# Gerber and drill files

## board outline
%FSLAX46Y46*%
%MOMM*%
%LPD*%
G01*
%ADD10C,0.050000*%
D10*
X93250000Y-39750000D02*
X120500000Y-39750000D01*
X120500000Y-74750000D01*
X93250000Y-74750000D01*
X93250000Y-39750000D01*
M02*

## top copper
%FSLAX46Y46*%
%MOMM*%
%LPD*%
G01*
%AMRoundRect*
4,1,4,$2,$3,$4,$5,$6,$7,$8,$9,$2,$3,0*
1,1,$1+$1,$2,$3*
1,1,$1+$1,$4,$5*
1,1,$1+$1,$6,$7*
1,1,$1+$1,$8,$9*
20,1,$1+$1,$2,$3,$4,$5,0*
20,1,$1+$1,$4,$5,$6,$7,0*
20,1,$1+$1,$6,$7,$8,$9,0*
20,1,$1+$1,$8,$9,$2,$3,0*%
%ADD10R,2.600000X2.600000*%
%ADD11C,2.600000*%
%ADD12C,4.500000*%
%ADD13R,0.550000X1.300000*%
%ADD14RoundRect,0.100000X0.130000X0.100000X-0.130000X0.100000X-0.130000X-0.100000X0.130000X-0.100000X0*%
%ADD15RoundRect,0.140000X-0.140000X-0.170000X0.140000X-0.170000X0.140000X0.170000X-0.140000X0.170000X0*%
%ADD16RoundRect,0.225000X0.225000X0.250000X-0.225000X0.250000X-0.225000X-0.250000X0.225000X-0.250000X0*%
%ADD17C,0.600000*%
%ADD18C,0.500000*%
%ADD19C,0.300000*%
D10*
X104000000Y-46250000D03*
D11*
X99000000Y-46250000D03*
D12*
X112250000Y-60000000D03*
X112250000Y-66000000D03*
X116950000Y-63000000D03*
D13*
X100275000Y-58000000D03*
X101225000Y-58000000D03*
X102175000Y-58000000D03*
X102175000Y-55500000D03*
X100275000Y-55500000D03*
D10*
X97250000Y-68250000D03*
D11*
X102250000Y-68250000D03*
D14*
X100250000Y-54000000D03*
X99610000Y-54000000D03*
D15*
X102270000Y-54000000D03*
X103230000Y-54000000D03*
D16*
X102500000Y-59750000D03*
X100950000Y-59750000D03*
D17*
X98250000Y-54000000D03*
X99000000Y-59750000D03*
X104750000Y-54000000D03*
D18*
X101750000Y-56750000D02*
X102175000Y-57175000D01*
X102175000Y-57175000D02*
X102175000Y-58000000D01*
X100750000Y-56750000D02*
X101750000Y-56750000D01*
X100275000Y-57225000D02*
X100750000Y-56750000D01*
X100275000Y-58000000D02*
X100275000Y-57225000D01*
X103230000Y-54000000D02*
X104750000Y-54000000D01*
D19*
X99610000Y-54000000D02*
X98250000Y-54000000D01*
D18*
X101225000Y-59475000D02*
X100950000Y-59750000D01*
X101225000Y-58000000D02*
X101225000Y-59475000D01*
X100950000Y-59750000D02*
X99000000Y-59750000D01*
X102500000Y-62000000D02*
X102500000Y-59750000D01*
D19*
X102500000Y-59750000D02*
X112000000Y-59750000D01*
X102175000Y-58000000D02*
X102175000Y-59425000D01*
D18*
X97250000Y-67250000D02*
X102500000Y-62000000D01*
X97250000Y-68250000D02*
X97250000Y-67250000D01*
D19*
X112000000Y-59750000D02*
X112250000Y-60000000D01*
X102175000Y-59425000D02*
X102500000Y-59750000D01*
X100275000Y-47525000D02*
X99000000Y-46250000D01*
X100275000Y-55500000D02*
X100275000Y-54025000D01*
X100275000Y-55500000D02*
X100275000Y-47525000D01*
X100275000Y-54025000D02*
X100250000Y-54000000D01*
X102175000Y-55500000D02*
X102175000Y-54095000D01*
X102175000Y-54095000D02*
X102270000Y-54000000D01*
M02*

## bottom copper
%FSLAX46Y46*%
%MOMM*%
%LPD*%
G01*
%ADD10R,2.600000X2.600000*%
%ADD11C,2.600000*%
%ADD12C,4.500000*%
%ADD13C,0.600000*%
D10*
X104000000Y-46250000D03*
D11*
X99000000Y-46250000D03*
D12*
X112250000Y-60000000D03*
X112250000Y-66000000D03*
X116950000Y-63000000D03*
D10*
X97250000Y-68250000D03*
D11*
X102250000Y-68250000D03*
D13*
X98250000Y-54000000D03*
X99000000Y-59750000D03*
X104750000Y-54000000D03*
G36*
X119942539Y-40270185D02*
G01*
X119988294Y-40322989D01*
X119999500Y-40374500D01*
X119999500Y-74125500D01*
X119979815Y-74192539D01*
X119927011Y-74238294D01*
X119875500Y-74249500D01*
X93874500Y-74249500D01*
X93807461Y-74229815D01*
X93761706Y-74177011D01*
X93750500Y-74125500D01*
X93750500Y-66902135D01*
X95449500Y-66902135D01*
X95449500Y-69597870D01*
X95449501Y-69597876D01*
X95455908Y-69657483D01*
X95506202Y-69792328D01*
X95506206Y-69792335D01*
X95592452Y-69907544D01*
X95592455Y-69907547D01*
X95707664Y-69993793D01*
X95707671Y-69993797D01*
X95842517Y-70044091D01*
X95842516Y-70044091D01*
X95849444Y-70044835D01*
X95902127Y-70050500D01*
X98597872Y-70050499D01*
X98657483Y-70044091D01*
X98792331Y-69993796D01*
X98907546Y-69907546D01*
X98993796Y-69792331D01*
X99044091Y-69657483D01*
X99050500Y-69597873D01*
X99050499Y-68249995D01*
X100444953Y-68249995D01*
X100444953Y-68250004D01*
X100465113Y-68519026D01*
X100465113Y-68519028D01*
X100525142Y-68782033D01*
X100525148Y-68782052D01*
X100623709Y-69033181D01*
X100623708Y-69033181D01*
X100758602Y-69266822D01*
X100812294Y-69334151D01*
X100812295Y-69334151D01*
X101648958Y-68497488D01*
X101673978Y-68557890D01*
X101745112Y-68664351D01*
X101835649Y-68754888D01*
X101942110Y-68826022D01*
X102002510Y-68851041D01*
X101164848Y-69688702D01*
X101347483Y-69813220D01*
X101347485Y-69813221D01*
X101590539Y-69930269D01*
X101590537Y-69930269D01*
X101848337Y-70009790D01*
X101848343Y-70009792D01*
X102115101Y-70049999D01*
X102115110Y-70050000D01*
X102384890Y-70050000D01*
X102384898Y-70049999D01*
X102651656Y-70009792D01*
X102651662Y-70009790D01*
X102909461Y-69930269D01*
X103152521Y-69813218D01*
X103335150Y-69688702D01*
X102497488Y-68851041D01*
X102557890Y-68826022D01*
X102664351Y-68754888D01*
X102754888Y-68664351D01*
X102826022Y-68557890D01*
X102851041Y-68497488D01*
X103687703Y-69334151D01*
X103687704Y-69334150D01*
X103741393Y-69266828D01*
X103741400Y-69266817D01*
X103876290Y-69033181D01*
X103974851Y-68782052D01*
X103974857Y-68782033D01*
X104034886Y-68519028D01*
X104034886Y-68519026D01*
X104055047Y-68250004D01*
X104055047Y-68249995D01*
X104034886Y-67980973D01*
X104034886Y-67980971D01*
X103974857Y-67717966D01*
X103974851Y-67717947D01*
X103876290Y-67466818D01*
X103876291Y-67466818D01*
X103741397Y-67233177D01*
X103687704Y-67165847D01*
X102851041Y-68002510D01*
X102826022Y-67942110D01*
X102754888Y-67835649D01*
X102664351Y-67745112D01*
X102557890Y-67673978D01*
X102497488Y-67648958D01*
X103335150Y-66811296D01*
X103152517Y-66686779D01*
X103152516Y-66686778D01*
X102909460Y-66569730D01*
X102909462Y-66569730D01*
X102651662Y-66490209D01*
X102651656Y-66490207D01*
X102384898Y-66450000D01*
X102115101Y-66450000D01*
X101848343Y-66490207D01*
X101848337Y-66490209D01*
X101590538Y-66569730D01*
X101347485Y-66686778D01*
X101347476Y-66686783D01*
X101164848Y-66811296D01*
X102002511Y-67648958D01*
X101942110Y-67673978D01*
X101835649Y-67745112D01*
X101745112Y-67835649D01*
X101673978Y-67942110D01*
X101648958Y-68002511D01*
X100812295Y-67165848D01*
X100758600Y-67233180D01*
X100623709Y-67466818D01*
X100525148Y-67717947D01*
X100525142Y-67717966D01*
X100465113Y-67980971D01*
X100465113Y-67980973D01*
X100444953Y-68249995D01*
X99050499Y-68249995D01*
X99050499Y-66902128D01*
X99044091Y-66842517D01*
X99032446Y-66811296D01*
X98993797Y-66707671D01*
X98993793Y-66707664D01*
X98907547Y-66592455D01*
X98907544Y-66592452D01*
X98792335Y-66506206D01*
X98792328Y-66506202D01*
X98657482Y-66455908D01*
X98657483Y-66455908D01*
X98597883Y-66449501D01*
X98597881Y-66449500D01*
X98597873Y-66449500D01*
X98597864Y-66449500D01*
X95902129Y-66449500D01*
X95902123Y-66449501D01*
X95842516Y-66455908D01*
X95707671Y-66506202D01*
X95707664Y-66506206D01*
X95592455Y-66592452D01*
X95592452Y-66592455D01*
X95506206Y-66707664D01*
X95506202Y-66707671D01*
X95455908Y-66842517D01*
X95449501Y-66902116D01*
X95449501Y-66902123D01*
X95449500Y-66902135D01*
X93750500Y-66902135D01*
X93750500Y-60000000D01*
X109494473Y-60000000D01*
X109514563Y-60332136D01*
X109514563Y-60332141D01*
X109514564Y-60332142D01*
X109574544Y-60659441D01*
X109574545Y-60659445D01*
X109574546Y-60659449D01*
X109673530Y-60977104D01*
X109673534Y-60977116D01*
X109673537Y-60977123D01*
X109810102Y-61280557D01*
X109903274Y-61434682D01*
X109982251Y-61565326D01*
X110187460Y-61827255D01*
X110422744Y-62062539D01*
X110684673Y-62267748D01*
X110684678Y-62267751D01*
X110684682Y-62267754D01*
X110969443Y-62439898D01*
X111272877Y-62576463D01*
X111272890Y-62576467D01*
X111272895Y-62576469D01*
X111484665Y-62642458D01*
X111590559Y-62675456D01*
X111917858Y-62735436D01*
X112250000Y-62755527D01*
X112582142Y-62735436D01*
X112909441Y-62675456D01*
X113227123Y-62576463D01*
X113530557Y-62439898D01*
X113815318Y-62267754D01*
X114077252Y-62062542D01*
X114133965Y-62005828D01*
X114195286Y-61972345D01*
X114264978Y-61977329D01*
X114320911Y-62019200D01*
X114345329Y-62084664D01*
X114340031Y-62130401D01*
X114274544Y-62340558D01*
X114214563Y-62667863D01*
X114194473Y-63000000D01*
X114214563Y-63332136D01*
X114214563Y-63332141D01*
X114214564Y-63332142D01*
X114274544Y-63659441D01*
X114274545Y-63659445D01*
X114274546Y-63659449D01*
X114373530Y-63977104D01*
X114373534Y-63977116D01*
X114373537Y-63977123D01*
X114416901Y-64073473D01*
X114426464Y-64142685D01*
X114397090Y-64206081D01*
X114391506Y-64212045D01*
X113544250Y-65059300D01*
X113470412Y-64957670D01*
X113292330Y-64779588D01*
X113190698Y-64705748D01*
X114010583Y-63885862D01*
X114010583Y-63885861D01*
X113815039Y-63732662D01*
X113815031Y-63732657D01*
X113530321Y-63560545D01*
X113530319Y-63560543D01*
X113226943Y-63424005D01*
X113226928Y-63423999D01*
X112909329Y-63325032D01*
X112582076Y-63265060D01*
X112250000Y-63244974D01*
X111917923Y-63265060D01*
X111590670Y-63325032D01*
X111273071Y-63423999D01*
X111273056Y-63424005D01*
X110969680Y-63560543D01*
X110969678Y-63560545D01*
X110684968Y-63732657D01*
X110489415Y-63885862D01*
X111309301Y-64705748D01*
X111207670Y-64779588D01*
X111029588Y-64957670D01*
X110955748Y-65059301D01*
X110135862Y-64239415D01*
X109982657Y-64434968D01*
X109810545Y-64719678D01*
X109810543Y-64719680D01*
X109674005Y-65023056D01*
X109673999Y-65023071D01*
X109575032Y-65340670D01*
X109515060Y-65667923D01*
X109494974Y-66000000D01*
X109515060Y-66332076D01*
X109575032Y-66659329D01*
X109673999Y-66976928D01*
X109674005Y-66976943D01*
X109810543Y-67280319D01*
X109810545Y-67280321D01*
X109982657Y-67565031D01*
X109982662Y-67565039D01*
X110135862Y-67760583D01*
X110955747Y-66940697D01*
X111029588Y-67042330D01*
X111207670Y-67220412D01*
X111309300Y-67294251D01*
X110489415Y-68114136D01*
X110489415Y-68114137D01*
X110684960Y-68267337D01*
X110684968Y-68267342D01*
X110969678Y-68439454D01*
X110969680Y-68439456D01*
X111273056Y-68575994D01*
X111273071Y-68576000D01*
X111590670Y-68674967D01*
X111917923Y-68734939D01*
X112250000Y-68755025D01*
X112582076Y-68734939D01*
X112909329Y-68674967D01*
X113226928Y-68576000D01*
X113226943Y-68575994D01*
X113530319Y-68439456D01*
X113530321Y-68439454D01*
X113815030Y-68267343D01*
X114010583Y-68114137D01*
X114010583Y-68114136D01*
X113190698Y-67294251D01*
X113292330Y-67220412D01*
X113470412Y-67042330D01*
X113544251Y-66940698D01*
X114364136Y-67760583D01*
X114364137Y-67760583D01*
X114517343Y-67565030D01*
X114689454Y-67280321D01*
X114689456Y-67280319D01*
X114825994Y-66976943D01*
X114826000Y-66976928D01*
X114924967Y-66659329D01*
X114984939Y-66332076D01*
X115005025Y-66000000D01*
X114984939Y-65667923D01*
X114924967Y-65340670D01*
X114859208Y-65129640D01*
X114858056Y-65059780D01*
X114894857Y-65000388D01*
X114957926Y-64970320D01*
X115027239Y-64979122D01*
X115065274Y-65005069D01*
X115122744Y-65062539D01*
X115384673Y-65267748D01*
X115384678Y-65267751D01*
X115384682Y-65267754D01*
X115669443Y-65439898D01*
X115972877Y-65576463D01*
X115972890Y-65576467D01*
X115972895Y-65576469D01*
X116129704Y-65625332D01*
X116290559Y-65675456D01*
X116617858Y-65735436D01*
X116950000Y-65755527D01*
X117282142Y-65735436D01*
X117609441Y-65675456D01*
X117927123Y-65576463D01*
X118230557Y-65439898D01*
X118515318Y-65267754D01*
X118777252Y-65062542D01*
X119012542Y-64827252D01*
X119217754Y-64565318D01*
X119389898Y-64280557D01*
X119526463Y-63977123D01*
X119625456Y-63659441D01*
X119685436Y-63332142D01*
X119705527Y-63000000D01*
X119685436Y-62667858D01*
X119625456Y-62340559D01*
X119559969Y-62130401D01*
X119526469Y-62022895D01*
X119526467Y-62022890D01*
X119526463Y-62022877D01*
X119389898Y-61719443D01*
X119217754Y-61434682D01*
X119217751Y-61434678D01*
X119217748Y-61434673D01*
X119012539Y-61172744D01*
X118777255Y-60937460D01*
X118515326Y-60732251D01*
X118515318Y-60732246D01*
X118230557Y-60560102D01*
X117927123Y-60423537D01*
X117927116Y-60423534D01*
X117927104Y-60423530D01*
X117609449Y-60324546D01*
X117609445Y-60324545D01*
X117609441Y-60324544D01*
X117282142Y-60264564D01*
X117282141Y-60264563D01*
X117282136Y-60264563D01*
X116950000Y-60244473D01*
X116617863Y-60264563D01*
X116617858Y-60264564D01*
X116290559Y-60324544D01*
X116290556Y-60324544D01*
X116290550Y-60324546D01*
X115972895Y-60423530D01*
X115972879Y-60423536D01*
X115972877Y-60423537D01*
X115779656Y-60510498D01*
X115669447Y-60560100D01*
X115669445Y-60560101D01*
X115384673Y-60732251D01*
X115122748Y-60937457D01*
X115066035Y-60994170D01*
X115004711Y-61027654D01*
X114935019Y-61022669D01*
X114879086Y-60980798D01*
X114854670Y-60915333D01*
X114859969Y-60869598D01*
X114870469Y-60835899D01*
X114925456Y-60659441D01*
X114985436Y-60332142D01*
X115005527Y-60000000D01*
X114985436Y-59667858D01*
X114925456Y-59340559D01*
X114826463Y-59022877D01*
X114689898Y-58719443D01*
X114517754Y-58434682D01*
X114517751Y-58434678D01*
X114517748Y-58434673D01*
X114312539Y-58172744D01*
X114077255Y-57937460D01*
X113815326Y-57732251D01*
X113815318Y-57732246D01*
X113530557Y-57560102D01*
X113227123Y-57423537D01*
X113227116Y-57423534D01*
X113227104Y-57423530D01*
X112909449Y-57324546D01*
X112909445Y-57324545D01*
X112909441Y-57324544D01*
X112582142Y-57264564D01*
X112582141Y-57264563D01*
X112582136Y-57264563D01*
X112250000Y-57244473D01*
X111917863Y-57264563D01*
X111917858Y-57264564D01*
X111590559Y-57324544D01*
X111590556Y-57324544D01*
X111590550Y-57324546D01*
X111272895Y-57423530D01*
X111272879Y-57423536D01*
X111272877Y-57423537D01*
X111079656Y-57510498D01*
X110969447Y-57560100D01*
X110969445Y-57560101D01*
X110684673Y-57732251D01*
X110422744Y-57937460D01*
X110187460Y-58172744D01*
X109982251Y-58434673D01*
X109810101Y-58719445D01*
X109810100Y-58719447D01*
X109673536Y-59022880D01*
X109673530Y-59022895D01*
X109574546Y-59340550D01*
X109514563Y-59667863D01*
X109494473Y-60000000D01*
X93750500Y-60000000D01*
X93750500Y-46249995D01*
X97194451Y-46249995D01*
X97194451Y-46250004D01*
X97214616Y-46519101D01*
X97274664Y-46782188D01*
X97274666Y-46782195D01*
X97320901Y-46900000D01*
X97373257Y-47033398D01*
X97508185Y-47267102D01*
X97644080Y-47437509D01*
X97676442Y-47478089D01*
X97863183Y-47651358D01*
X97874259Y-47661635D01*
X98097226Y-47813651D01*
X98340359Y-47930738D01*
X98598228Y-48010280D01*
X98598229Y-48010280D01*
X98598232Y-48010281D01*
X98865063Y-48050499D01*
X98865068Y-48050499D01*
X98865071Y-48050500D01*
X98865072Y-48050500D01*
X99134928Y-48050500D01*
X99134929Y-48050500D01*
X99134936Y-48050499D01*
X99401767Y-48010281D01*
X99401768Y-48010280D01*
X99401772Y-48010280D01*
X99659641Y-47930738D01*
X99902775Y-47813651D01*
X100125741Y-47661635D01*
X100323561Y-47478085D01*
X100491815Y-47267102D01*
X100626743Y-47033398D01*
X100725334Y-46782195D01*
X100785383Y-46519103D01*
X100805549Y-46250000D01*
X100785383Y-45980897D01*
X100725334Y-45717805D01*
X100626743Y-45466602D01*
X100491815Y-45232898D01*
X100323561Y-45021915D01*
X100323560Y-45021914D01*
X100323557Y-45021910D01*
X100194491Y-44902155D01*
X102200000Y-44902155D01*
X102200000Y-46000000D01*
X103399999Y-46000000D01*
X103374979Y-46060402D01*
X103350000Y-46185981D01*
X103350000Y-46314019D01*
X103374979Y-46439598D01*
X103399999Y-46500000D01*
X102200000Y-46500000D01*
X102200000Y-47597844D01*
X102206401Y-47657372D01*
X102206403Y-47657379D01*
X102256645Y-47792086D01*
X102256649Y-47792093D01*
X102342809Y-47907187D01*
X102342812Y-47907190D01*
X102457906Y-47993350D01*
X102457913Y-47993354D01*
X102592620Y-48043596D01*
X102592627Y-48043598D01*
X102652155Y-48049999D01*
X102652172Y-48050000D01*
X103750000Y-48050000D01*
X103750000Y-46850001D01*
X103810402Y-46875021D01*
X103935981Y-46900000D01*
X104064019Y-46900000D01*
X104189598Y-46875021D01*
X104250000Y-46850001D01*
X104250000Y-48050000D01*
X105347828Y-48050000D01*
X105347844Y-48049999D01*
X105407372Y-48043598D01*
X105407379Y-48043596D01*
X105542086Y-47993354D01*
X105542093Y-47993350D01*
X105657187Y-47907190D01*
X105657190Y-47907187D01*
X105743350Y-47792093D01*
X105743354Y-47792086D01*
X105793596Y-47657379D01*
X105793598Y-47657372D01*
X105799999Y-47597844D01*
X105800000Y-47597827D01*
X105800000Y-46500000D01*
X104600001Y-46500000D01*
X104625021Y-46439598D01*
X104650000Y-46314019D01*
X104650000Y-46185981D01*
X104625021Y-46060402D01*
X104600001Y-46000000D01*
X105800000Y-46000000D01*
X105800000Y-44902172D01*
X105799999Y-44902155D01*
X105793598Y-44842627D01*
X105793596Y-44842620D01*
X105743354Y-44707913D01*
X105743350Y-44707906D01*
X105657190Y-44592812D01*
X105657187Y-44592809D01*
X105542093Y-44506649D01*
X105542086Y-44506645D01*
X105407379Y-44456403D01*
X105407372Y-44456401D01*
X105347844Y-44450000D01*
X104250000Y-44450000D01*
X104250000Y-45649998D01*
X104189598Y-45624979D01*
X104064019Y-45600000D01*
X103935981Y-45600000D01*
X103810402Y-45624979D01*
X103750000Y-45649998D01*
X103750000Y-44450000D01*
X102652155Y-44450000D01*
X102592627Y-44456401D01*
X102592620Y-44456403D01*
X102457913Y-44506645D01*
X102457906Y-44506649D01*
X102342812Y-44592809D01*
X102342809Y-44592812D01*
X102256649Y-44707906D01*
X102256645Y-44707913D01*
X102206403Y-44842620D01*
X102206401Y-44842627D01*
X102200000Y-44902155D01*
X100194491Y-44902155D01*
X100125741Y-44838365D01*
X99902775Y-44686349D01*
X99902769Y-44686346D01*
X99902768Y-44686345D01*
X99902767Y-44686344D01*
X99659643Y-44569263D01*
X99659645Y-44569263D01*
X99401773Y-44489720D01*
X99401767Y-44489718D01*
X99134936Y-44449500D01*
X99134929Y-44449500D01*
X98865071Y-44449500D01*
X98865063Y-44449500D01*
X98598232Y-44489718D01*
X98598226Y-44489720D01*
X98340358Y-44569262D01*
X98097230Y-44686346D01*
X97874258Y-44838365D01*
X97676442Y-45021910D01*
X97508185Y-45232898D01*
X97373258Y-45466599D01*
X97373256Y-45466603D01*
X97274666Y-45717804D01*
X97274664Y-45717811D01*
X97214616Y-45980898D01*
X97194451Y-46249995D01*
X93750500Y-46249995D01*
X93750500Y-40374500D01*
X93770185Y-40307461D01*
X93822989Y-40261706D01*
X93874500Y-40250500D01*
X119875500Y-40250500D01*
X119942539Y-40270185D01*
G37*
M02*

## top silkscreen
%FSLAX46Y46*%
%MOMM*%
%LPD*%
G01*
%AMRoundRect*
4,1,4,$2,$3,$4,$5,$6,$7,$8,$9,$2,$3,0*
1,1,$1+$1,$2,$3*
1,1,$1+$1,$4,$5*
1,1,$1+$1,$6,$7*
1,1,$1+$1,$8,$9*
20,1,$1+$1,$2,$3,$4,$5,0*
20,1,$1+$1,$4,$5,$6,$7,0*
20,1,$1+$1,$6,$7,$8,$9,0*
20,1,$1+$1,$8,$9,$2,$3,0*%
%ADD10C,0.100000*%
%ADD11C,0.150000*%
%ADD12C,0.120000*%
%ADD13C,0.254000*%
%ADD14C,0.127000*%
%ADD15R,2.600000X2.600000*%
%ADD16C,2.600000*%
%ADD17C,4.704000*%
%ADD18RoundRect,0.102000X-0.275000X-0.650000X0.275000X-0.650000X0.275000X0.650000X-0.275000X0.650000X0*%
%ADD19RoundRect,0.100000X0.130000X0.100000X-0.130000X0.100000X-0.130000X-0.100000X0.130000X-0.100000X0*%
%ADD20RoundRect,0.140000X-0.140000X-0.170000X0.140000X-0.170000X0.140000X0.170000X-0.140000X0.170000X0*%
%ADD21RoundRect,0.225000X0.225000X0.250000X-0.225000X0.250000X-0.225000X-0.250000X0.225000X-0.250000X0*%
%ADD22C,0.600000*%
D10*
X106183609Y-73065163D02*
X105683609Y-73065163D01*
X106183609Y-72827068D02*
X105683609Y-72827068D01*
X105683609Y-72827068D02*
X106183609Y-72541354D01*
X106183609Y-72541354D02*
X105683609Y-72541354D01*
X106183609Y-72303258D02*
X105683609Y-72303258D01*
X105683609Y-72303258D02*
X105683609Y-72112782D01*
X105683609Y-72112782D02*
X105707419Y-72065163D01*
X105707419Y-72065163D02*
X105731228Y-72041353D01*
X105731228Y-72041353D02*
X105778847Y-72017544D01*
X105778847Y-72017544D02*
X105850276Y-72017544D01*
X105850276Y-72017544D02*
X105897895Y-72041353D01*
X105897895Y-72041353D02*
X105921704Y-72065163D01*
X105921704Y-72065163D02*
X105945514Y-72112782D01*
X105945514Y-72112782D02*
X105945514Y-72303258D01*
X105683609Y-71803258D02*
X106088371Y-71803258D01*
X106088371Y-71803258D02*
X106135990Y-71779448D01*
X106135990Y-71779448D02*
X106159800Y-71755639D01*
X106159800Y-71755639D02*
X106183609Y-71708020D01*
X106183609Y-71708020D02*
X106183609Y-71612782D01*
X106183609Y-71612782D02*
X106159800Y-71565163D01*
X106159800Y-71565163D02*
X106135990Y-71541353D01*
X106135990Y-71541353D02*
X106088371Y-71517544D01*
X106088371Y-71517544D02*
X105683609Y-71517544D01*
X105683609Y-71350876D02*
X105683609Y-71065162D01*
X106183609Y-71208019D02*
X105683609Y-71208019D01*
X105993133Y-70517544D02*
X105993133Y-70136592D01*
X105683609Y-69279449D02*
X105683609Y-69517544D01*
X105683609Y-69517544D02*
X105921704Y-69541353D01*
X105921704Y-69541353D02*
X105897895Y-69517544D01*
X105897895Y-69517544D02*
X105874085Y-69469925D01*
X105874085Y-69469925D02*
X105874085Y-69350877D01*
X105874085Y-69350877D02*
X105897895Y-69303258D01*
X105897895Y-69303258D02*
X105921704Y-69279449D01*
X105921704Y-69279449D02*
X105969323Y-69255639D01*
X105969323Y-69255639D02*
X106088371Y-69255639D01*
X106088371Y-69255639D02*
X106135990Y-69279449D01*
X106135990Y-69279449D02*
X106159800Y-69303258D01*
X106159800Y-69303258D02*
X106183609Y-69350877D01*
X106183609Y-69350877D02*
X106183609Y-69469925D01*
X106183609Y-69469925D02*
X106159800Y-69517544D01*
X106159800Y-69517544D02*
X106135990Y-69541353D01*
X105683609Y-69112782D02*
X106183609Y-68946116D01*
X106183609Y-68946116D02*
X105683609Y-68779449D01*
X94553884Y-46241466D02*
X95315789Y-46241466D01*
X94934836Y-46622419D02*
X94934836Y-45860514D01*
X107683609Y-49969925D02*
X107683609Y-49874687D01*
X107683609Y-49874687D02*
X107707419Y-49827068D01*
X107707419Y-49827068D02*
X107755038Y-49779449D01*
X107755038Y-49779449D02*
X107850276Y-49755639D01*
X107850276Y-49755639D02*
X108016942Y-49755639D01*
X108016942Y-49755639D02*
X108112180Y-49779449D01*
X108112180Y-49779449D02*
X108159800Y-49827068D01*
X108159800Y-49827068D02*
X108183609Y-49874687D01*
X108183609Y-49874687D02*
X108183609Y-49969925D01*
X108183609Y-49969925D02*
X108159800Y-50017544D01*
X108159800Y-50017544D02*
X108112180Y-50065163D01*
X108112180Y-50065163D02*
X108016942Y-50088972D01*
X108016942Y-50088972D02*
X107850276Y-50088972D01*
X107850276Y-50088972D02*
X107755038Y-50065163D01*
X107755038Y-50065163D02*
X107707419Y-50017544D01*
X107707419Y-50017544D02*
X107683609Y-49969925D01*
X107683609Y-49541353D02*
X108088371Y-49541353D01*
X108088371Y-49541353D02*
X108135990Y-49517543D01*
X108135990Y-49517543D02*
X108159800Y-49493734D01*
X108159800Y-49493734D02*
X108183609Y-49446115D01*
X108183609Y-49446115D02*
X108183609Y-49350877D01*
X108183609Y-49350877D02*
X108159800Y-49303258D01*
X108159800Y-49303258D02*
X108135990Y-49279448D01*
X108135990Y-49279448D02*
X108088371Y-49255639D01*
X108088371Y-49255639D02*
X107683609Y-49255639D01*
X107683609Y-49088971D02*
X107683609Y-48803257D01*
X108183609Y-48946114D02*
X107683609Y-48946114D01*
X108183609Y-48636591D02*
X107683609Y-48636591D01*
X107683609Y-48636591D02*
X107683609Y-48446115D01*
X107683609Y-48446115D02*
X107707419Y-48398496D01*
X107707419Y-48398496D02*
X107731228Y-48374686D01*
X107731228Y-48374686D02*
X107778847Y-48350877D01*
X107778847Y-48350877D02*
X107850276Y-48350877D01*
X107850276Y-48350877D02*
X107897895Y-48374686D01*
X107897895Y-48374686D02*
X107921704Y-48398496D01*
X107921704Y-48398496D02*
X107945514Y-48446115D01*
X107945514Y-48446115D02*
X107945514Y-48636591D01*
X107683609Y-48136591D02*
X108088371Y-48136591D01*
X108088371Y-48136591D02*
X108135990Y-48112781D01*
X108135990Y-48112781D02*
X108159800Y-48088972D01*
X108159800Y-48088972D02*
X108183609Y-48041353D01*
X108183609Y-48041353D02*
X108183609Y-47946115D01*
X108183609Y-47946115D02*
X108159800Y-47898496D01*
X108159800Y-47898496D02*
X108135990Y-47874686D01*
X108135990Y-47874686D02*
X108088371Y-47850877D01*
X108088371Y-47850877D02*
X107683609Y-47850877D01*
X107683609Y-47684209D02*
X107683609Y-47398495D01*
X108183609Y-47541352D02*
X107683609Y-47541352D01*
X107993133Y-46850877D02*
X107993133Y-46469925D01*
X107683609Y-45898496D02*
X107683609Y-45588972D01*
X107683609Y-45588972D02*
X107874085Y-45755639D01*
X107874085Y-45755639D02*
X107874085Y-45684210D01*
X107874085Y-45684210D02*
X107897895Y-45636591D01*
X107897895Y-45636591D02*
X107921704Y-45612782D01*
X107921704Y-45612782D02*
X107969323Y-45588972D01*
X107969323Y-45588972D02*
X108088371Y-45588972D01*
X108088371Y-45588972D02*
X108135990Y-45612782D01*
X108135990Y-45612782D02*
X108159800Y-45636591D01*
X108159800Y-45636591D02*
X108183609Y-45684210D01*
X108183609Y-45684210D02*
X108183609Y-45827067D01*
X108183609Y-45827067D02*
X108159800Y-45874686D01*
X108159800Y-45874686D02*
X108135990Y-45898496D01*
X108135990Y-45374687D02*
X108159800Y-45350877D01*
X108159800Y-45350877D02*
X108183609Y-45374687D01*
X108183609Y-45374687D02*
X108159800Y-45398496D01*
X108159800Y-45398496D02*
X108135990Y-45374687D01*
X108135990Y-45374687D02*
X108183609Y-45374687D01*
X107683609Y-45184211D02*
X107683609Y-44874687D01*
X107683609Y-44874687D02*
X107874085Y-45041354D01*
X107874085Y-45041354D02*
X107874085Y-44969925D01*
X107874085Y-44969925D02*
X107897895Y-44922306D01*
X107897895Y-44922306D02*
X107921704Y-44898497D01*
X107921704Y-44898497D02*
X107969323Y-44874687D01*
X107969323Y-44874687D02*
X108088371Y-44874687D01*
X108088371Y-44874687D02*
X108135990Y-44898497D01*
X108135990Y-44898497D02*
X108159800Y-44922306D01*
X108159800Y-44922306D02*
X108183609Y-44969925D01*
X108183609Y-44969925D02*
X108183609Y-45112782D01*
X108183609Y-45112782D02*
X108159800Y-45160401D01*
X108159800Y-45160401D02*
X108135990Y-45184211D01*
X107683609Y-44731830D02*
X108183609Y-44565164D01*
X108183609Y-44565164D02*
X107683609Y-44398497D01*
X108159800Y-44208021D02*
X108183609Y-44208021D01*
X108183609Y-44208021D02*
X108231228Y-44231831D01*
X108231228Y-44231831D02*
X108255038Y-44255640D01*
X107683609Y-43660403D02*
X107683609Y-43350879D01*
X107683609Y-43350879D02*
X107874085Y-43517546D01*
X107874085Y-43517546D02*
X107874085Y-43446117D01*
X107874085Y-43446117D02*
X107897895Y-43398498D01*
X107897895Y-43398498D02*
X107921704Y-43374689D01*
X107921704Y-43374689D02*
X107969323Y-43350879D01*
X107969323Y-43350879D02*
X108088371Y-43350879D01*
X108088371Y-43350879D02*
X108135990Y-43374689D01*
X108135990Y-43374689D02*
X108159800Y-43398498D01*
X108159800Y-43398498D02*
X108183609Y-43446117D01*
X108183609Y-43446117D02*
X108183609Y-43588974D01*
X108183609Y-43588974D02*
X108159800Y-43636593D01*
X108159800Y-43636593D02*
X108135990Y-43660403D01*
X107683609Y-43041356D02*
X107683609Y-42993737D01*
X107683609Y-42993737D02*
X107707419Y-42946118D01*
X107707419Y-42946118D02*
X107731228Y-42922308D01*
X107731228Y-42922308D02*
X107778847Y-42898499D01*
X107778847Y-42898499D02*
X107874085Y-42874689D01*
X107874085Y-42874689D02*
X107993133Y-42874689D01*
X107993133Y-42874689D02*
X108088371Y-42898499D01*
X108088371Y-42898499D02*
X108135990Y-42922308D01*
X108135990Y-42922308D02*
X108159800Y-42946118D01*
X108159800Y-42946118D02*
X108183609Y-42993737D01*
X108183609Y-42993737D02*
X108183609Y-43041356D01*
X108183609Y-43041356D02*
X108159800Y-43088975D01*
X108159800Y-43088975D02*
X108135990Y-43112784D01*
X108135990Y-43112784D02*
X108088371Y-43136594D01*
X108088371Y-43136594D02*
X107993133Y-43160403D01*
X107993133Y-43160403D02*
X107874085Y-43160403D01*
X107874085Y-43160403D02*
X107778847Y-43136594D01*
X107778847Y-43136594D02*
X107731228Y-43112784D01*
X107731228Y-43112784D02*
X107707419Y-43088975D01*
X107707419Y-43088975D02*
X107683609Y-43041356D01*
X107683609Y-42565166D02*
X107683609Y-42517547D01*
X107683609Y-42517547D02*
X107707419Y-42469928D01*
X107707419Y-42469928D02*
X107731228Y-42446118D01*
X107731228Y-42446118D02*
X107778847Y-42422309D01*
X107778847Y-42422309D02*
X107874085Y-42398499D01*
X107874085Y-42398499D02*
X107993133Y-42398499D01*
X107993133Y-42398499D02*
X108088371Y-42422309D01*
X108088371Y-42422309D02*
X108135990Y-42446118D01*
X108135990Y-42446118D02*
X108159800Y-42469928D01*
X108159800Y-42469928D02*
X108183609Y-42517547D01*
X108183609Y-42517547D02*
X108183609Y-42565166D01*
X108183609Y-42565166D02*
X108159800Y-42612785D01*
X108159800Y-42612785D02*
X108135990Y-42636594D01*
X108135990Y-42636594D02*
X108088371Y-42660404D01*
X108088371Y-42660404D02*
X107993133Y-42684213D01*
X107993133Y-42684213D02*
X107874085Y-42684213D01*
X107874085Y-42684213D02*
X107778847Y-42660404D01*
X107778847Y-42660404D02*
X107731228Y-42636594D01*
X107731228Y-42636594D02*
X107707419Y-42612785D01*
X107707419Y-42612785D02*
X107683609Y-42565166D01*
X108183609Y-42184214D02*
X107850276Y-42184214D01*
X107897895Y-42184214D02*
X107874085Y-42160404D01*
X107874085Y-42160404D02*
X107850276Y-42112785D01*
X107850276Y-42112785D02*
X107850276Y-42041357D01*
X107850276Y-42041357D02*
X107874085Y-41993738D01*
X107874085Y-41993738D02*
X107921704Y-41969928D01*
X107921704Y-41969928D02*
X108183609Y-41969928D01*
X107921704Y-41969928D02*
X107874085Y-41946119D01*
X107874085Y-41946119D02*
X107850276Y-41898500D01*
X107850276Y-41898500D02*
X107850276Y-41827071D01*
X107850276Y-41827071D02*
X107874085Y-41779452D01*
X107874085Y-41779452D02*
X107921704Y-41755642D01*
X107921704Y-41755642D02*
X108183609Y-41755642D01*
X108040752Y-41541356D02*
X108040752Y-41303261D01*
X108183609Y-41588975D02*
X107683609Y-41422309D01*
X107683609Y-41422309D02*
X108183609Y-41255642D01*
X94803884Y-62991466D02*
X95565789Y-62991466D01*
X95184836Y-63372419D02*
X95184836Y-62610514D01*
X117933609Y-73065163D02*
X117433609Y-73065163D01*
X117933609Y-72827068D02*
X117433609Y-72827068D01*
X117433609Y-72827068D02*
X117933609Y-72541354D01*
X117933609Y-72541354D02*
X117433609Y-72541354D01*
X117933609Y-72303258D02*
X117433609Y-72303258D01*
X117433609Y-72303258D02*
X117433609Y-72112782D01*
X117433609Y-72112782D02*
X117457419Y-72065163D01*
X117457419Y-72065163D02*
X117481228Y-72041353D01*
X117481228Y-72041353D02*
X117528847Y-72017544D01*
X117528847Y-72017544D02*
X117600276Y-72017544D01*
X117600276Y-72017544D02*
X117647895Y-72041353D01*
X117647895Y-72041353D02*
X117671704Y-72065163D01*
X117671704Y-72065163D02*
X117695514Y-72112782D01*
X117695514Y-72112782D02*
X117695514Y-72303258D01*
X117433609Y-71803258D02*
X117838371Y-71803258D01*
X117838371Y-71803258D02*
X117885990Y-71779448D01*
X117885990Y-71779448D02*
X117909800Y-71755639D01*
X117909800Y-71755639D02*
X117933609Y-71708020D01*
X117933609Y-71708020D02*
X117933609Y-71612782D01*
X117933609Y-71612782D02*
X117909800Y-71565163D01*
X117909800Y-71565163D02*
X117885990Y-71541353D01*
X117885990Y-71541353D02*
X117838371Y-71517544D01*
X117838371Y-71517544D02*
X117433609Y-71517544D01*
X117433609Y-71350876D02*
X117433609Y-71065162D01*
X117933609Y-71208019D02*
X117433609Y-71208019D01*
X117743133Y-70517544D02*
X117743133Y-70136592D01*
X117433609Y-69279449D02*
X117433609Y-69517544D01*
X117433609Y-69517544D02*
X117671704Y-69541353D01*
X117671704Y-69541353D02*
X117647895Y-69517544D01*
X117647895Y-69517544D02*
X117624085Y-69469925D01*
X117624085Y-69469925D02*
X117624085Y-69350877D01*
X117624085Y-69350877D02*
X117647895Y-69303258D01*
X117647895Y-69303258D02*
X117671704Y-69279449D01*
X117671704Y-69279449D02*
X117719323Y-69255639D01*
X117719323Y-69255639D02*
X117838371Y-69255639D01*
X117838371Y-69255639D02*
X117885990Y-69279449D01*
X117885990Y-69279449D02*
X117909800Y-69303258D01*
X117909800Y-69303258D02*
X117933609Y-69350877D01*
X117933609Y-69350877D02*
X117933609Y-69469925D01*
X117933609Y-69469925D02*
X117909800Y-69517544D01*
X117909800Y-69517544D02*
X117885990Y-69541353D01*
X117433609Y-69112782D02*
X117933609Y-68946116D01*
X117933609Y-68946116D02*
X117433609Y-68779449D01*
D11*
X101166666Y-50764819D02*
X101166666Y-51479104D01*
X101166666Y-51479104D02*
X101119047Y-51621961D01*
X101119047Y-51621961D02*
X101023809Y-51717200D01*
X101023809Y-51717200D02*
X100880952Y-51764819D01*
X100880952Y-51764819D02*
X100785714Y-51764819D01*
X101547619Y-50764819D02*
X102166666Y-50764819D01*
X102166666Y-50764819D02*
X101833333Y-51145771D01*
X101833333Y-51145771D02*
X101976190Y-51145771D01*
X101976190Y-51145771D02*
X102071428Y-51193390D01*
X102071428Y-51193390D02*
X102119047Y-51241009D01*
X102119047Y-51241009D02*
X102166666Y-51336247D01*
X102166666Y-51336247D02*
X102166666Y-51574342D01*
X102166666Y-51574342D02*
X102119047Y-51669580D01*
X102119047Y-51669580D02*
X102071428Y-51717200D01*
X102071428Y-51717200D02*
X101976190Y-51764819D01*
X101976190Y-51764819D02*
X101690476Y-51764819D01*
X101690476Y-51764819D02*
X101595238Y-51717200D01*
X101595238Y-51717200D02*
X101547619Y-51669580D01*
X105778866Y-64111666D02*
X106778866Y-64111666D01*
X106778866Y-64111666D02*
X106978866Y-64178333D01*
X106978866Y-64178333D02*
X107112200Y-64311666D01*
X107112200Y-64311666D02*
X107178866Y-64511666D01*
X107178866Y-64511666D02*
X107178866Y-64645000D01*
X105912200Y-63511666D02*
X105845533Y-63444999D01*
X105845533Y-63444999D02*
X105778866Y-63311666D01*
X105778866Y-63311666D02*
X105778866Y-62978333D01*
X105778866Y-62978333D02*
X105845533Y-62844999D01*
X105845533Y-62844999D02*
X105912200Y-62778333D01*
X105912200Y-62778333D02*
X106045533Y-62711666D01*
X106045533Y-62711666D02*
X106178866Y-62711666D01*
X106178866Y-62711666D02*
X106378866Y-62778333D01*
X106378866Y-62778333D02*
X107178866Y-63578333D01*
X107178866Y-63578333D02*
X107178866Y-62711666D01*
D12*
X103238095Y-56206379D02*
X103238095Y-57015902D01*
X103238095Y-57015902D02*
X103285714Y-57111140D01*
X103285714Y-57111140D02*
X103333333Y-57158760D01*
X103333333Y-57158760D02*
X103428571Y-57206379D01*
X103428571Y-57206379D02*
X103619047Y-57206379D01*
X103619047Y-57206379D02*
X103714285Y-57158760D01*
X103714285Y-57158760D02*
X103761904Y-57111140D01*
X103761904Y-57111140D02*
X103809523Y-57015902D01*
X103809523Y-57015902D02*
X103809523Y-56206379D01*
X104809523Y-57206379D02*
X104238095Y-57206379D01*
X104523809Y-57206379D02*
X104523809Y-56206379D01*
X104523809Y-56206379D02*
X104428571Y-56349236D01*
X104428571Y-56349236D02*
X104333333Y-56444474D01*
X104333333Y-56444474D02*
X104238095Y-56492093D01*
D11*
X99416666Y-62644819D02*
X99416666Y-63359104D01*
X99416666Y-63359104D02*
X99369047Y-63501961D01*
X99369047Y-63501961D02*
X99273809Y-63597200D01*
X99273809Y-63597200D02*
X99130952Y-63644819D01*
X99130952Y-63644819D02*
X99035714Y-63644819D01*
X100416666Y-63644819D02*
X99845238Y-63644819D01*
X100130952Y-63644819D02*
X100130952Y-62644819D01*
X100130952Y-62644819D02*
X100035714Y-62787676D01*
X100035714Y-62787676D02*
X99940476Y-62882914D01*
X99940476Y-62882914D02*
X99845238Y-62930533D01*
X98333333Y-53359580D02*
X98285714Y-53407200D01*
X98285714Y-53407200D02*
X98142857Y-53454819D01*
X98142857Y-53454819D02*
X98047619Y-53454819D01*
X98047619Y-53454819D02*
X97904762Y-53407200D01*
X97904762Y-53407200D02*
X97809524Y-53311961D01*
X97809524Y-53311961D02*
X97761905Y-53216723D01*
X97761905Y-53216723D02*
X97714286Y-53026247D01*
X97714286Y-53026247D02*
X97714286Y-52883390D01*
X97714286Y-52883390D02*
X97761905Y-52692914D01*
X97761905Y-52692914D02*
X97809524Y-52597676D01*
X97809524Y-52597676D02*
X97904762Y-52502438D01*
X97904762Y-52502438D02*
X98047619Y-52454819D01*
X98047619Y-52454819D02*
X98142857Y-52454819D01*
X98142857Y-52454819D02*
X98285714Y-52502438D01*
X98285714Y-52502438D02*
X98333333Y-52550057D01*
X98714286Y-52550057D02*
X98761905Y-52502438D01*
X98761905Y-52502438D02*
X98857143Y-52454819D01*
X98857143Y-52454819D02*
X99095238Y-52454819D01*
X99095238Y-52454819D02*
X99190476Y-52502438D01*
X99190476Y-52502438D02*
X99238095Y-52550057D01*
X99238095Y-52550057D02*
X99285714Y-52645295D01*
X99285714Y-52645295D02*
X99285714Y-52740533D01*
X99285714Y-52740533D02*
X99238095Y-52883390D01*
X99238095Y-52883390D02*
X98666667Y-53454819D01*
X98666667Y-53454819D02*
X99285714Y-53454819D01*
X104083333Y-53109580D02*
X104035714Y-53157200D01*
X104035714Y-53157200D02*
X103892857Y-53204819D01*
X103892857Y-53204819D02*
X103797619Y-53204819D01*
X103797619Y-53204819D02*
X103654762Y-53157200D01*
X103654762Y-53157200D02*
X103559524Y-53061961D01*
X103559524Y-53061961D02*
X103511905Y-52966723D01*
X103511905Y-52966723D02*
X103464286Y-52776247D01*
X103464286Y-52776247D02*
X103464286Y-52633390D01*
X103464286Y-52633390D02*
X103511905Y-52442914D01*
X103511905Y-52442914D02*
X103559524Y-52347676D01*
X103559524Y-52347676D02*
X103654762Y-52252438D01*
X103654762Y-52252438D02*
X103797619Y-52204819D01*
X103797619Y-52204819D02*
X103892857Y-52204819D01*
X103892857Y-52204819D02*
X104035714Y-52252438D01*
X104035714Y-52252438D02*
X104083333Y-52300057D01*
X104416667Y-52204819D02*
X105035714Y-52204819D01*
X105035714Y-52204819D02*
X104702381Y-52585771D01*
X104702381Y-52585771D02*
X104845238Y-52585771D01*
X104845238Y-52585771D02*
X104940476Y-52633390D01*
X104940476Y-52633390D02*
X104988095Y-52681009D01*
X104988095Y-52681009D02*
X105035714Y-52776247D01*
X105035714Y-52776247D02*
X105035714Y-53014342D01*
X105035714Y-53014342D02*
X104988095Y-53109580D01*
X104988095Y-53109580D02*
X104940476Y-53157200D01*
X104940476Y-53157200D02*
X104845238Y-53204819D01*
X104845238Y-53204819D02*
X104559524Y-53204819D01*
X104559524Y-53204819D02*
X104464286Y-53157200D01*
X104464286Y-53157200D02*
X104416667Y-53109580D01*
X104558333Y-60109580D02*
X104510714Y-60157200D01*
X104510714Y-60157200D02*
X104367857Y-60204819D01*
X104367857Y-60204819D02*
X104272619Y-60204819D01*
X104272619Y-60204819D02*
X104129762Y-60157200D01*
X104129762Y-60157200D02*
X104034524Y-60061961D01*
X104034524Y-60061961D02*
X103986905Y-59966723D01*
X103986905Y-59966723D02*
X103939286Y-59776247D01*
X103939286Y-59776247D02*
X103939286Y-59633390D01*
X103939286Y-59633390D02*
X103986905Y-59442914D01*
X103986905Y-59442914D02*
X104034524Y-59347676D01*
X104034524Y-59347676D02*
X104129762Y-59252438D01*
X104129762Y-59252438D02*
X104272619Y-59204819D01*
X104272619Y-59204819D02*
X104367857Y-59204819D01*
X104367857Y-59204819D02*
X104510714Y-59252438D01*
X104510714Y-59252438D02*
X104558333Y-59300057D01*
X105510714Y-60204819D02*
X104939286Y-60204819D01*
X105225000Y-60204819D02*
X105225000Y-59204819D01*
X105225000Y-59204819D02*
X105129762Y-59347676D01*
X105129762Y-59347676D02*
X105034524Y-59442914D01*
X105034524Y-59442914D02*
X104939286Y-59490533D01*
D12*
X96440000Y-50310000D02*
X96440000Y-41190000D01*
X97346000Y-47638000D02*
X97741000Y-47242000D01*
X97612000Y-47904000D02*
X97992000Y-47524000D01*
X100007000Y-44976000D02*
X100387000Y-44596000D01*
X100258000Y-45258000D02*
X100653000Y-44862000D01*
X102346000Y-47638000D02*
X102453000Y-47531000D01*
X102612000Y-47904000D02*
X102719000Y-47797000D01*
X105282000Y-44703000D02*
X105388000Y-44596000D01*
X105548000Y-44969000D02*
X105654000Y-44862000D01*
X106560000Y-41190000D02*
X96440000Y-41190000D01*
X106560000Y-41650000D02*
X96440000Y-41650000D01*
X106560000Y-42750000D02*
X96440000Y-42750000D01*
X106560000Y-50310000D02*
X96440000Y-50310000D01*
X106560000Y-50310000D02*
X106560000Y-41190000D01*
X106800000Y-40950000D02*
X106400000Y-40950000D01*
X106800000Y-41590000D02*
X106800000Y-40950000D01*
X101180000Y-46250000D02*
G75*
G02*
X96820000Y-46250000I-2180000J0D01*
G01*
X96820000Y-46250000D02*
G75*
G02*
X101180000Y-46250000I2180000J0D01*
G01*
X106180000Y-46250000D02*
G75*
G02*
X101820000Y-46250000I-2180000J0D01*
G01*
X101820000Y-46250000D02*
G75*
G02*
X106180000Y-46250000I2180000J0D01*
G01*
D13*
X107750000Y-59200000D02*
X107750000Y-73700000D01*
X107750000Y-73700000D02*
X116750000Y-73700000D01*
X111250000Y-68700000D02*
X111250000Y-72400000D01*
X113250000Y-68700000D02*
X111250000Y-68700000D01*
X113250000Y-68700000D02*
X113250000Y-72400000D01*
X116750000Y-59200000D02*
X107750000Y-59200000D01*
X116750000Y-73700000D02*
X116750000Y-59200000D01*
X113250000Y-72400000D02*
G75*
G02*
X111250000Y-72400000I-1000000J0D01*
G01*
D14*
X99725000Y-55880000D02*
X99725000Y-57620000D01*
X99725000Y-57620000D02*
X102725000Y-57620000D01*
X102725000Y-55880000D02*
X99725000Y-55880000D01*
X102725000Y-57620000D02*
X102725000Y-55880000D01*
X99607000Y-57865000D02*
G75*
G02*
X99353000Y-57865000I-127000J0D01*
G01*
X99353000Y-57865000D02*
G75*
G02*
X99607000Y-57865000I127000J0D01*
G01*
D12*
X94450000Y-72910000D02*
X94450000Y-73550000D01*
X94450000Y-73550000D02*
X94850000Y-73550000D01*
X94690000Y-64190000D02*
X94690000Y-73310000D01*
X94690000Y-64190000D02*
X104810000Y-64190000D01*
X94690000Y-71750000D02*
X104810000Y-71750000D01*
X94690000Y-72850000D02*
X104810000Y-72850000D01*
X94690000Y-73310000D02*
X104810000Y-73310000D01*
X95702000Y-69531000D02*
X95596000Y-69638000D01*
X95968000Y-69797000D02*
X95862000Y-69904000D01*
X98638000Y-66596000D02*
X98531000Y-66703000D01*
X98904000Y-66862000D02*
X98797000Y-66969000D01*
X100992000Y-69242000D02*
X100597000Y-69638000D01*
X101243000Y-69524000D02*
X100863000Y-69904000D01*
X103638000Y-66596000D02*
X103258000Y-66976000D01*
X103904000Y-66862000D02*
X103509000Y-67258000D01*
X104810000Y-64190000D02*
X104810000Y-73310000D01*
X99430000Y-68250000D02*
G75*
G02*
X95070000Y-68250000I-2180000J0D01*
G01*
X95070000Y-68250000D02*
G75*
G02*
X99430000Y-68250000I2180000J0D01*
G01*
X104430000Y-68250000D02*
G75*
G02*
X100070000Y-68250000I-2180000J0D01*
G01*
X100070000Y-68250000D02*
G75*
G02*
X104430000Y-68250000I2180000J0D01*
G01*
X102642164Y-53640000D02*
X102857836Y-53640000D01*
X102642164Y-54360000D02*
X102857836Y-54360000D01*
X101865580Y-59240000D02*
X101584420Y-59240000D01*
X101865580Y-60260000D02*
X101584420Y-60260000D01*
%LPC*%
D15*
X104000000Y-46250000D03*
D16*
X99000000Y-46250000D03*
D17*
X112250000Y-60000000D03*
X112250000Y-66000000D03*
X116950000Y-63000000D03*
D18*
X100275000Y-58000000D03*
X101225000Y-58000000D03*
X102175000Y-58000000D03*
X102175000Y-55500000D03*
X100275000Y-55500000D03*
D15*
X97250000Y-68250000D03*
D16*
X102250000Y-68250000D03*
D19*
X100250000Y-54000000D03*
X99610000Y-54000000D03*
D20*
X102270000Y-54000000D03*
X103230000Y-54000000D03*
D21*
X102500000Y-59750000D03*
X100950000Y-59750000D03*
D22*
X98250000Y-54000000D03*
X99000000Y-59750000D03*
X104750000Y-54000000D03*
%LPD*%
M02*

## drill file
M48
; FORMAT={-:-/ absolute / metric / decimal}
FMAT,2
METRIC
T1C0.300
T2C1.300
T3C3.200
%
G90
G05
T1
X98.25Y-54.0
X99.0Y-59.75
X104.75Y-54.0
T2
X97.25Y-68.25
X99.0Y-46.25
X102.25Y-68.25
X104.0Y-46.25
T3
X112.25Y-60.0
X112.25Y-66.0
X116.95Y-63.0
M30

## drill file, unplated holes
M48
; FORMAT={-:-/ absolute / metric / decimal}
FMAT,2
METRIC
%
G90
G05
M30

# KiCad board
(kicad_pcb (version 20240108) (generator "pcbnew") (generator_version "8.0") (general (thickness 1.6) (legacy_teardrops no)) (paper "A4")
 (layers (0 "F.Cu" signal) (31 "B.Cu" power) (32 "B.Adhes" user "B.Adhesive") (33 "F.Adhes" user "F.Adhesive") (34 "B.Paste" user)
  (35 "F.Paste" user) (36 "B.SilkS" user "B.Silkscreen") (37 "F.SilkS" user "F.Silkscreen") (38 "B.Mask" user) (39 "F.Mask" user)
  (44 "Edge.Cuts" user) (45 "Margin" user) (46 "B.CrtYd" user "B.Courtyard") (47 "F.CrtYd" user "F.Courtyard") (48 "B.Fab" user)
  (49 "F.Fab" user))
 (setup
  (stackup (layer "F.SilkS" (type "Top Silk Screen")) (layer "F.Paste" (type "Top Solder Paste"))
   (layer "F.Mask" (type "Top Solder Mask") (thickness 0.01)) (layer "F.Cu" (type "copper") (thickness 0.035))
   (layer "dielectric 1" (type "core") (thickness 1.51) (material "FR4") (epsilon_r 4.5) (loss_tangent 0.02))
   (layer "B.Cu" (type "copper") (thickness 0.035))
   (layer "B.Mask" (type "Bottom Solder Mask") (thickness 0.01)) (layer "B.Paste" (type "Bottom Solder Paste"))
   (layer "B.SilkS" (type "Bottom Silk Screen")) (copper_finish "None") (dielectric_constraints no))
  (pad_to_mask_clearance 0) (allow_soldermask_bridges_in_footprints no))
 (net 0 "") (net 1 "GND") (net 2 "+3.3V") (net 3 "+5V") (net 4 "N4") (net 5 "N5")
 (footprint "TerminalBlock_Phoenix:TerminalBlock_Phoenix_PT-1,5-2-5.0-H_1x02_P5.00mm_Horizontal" (layer "F.Cu") (at 104 46.25 180)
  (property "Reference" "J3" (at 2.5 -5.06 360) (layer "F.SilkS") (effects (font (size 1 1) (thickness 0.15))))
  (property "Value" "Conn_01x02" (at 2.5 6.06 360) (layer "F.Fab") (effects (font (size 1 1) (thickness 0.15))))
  (fp_line (start 7.56 -4.06) (end 7.56 5.06) (stroke (width 0.12) (type solid)) (layer "F.SilkS"))
  (fp_line (start 6.654 -1.388) (end 6.259 -0.992) (stroke (width 0.12) (type solid)) (layer "F.SilkS"))
  (fp_line (start 6.388 -1.654) (end 6.008 -1.274) (stroke (width 0.12) (type solid)) (layer "F.SilkS"))
  (fp_line (start 3.993 1.274) (end 3.613 1.654) (stroke (width 0.12) (type solid)) (layer "F.SilkS"))
  (fp_line (start 3.742 0.992) (end 3.347 1.388) (stroke (width 0.12) (type solid)) (layer "F.SilkS"))
  (fp_line (start 1.654 -1.388) (end 1.547 -1.281) (stroke (width 0.12) (type solid)) (layer "F.SilkS"))
  (fp_line (start 1.388 -1.654) (end 1.281 -1.547) (stroke (width 0.12) (type solid)) (layer "F.SilkS"))
  (fp_line (start -1.282 1.547) (end -1.388 1.654) (stroke (width 0.12) (type solid)) (layer "F.SilkS"))
  (fp_line (start -1.548 1.281) (end -1.654 1.388) (stroke (width 0.12) (type solid)) (layer "F.SilkS"))
  (fp_line (start -2.56 5.06) (end 7.56 5.06) (stroke (width 0.12) (type solid)) (layer "F.SilkS"))
  (fp_line (start -2.56 4.6) (end 7.56 4.6) (stroke (width 0.12) (type solid)) (layer "F.SilkS"))
  (fp_line (start -2.56 3.5) (end 7.56 3.5) (stroke (width 0.12) (type solid)) (layer "F.SilkS"))
  (fp_line (start -2.56 -4.06) (end 7.56 -4.06) (stroke (width 0.12) (type solid)) (layer "F.SilkS"))
  (fp_line (start -2.56 -4.06) (end -2.56 5.06) (stroke (width 0.12) (type solid)) (layer "F.SilkS"))
  (fp_line (start -2.8 5.3) (end -2.4 5.3) (stroke (width 0.12) (type solid)) (layer "F.SilkS"))
  (fp_line (start -2.8 4.66) (end -2.8 5.3) (stroke (width 0.12) (type solid)) (layer "F.SilkS"))
  (fp_circle (center 5 0) (end 7.18 0) (stroke (width 0.12) (type solid)) (fill none) (layer "F.SilkS"))
  (fp_circle (center 0 0) (end 2.18 0) (stroke (width 0.12) (type solid)) (fill none) (layer "F.SilkS"))
  (pad "1" thru_hole rect (at 0 0 180) (size 2.6 2.6) (drill 1.3) (layers "*.Cu" "*.Mask") (remove_unused_layers no) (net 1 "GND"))
  (pad "2" thru_hole circle (at 5 0 180) (size 2.6 2.6) (drill 1.3) (layers "*.Cu" "*.Mask") (remove_unused_layers no) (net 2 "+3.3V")))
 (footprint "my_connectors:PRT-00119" (layer "F.Cu") (at 112.25 73.7 -90)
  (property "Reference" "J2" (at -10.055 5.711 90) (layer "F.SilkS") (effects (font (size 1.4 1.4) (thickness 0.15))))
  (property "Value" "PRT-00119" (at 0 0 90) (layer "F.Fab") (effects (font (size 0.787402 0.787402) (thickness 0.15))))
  (fp_line (start -14.5 4.5) (end 0 4.5) (stroke (width 0.254) (type solid)) (layer "F.SilkS"))
  (fp_line (start 0 4.5) (end 0 -4.5) (stroke (width 0.254) (type solid)) (layer "F.SilkS"))
  (fp_line (start -5 1) (end -1.3 1) (stroke (width 0.254) (type solid)) (layer "F.SilkS"))
  (fp_line (start -5 -1) (end -5 1) (stroke (width 0.254) (type solid)) (layer "F.SilkS"))
  (fp_line (start -5 -1) (end -1.3 -1) (stroke (width 0.254) (type solid)) (layer "F.SilkS"))
  (fp_line (start -14.5 -4.5) (end -14.5 4.5) (stroke (width 0.254) (type solid)) (layer "F.SilkS"))
  (fp_line (start 0 -4.5) (end -14.5 -4.5) (stroke (width 0.254) (type solid)) (layer "F.SilkS"))
  (fp_arc (start -1.3 -1) (mid -0.3 0) (end -1.3 1) (stroke (width 0.254) (type solid)) (layer "F.SilkS"))
  (pad "1" thru_hole circle (at -13.7 0 270) (size 4.5 4.5) (drill 3.2) (layers "*.Cu" "*.Mask") (remove_unused_layers no) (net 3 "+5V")
   (solder_mask_margin 0.102))
  (pad "2" thru_hole circle (at -7.7 0 270) (size 4.5 4.5) (drill 3.2) (layers "*.Cu" "*.Mask") (remove_unused_layers no) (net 1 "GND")
   (solder_mask_margin 0.102))
  (pad "3" thru_hole circle (at -10.7 -4.7 270) (size 4.5 4.5) (drill 3.2) (layers "*.Cu" "*.Mask") (remove_unused_layers no) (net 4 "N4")
   (solder_mask_margin 0.102)))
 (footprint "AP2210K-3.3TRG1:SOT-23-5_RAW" (layer "F.Cu") (at 101.225 56.75)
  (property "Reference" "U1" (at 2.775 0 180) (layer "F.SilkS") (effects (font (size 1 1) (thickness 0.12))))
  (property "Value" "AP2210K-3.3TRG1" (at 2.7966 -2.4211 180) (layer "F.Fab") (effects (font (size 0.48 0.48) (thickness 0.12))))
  (fp_line (start -1.5 -0.87) (end -1.5 0.87) (stroke (width 0.127) (type solid)) (layer "F.SilkS"))
  (fp_line (start -1.5 0.87) (end 1.5 0.87) (stroke (width 0.127) (type solid)) (layer "F.SilkS"))
  (fp_line (start 1.5 -0.87) (end -1.5 -0.87) (stroke (width 0.127) (type solid)) (layer "F.SilkS"))
  (fp_line (start 1.5 0.87) (end 1.5 -0.87) (stroke (width 0.127) (type solid)) (layer "F.SilkS"))
  (fp_circle (center -1.745 1.115) (end -1.618 1.115) (stroke (width 0.127) (type solid)) (fill none) (layer "F.SilkS"))
  (pad "1" smd rect (at -0.95 1.25) (size 0.55 1.3) (layers "F.Cu" "F.Paste" "F.Mask") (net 3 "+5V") (solder_mask_margin 0.102))
  (pad "2" smd rect (at 0 1.25) (size 0.55 1.3) (layers "F.Cu" "F.Paste" "F.Mask") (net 1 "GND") (solder_mask_margin 0.102))
  (pad "3" smd rect (at 0.95 1.25) (size 0.55 1.3) (layers "F.Cu" "F.Paste" "F.Mask") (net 3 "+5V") (solder_mask_margin 0.102))
  (pad "4" smd rect (at 0.95 -1.25) (size 0.55 1.3) (layers "F.Cu" "F.Paste" "F.Mask") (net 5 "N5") (solder_mask_margin 0.102))
  (pad "5" smd rect (at -0.95 -1.25) (size 0.55 1.3) (layers "F.Cu" "F.Paste" "F.Mask") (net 2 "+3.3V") (solder_mask_margin 0.102)))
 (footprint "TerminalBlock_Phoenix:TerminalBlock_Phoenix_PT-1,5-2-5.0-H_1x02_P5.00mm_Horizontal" (layer "F.Cu") (at 97.25 68.25)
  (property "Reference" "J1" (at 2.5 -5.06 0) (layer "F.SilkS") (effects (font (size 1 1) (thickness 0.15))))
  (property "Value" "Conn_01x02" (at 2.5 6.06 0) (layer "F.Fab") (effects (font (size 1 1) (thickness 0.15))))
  (fp_line (start -2.8 4.66) (end -2.8 5.3) (stroke (width 0.12) (type solid)) (layer "F.SilkS"))
  (fp_line (start -2.8 5.3) (end -2.4 5.3) (stroke (width 0.12) (type solid)) (layer "F.SilkS"))
  (fp_line (start -2.56 -4.06) (end -2.56 5.06) (stroke (width 0.12) (type solid)) (layer "F.SilkS"))
  (fp_line (start -2.56 -4.06) (end 7.56 -4.06) (stroke (width 0.12) (type solid)) (layer "F.SilkS"))
  (fp_line (start -2.56 3.5) (end 7.56 3.5) (stroke (width 0.12) (type solid)) (layer "F.SilkS"))
  (fp_line (start -2.56 4.6) (end 7.56 4.6) (stroke (width 0.12) (type solid)) (layer "F.SilkS"))
  (fp_line (start -2.56 5.06) (end 7.56 5.06) (stroke (width 0.12) (type solid)) (layer "F.SilkS"))
  (fp_line (start -1.548 1.281) (end -1.654 1.388) (stroke (width 0.12) (type solid)) (layer "F.SilkS"))
  (fp_line (start -1.282 1.547) (end -1.388 1.654) (stroke (width 0.12) (type solid)) (layer "F.SilkS"))
  (fp_line (start 1.388 -1.654) (end 1.281 -1.547) (stroke (width 0.12) (type solid)) (layer "F.SilkS"))
  (fp_line (start 1.654 -1.388) (end 1.547 -1.281) (stroke (width 0.12) (type solid)) (layer "F.SilkS"))
  (fp_line (start 3.742 0.992) (end 3.347 1.388) (stroke (width 0.12) (type solid)) (layer "F.SilkS"))
  (fp_line (start 3.993 1.274) (end 3.613 1.654) (stroke (width 0.12) (type solid)) (layer "F.SilkS"))
  (fp_line (start 6.388 -1.654) (end 6.008 -1.274) (stroke (width 0.12) (type solid)) (layer "F.SilkS"))
  (fp_line (start 6.654 -1.388) (end 6.259 -0.992) (stroke (width 0.12) (type solid)) (layer "F.SilkS"))
  (fp_line (start 7.56 -4.06) (end 7.56 5.06) (stroke (width 0.12) (type solid)) (layer "F.SilkS"))
  (fp_circle (center 0 0) (end 2.18 0) (stroke (width 0.12) (type solid)) (fill none) (layer "F.SilkS"))
  (fp_circle (center 5 0) (end 7.18 0) (stroke (width 0.12) (type solid)) (fill none) (layer "F.SilkS"))
  (pad "1" thru_hole rect (at 0 0) (size 2.6 2.6) (drill 1.3) (layers "*.Cu" "*.Mask") (remove_unused_layers no) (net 3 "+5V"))
  (pad "2" thru_hole circle (at 5 0) (size 2.6 2.6) (drill 1.3) (layers "*.Cu" "*.Mask") (remove_unused_layers no) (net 1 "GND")))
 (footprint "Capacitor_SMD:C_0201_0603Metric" (layer "F.Cu") (at 99.93 54 180)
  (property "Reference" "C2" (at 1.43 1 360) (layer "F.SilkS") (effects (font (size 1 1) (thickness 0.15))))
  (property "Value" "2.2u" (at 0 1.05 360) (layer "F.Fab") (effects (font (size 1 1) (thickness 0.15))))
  (pad "" smd roundrect (at -0.345 0 180) (size 0.318 0.36) (layers "F.Paste") (roundrect_rratio 0.25))
  (pad "" smd roundrect (at 0.345 0 180) (size 0.318 0.36) (layers "F.Paste") (roundrect_rratio 0.25))
  (pad "1" smd roundrect (at -0.32 0 180) (size 0.46 0.4) (layers "F.Cu" "F.Mask") (roundrect_rratio 0.25) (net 2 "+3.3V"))
  (pad "2" smd roundrect (at 0.32 0 180) (size 0.46 0.4) (layers "F.Cu" "F.Mask") (roundrect_rratio 0.25) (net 1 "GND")))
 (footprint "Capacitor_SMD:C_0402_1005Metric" (layer "F.Cu") (at 102.75 54)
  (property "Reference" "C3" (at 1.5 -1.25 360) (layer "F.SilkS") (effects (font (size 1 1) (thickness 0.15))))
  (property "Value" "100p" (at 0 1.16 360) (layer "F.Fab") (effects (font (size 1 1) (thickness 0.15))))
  (fp_line (start -0.107836 -0.36) (end 0.107836 -0.36) (stroke (width 0.12) (type solid)) (layer "F.SilkS"))
  (fp_line (start -0.107836 0.36) (end 0.107836 0.36) (stroke (width 0.12) (type solid)) (layer "F.SilkS"))
  (pad "1" smd roundrect (at -0.48 0) (size 0.56 0.62) (layers "F.Cu" "F.Paste" "F.Mask") (roundrect_rratio 0.25) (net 5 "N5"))
  (pad "2" smd roundrect (at 0.48 0) (size 0.56 0.62) (layers "F.Cu" "F.Paste" "F.Mask") (roundrect_rratio 0.25) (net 1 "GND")))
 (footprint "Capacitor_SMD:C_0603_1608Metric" (layer "F.Cu") (at 101.725 59.75 180)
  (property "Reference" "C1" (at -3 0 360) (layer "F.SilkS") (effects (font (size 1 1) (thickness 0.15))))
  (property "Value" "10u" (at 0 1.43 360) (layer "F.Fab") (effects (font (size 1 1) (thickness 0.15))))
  (fp_line (start -0.14058 0.51) (end 0.14058 0.51) (stroke (width 0.12) (type solid)) (layer "F.SilkS"))
  (fp_line (start -0.14058 -0.51) (end 0.14058 -0.51) (stroke (width 0.12) (type solid)) (layer "F.SilkS"))
  (pad "1" smd roundrect (at -0.775 0 180) (size 0.9 0.95) (layers "F.Cu" "F.Paste" "F.Mask") (roundrect_rratio 0.25) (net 3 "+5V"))
  (pad "2" smd roundrect (at 0.775 0 180) (size 0.9 0.95) (layers "F.Cu" "F.Paste" "F.Mask") (roundrect_rratio 0.25) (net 1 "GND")))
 (gr_rect (start 93.25 39.75) (end 120.5 74.75) (stroke (width 0.05) (type default)) (fill none) (layer "Edge.Cuts"))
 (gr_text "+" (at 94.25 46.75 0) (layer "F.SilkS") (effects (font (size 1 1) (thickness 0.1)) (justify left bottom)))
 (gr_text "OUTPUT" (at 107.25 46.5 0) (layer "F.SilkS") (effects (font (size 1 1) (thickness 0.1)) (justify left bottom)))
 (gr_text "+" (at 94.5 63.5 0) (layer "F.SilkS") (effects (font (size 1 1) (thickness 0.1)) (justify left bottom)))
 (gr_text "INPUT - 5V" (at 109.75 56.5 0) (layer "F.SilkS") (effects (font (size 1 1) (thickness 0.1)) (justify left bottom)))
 (segment (start 103.23 54) (end 104.75 54) (width 0.5) (layer "F.Cu") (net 1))
 (segment (start 99.61 54) (end 98.25 54) (width 0.3) (layer "F.Cu") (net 1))
 (segment (start 101.225 59.475) (end 100.95 59.75) (width 0.5) (layer "F.Cu") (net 1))
 (segment (start 101.225 58) (end 101.225 59.475) (width 0.5) (layer "F.Cu") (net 1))
 (segment (start 100.95 59.75) (end 99 59.75) (width 0.5) (layer "F.Cu") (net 1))
 (via (at 98.25 54) (size 0.6) (drill 0.3) (layers "F.Cu" "B.Cu") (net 1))
 (via (at 99 59.75) (size 0.6) (drill 0.3) (layers "F.Cu" "B.Cu") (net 1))
 (via (at 104.75 54) (size 0.6) (drill 0.3) (layers "F.Cu" "B.Cu") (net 1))
 (segment (start 102.5 62) (end 102.5 59.75) (width 0.5) (layer "F.Cu") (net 3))
 (segment (start 100.275 57.225) (end 100.75 56.75) (width 0.3) (layer "F.Cu") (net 3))
 (segment (start 102.5 59.75) (end 112 59.75) (width 0.3) (layer "F.Cu") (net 3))
 (segment (start 100.275 58) (end 100.275 57.225) (width 0.3) (layer "F.Cu") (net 3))
 (segment (start 102.175 58) (end 102.175 59.425) (width 0.3) (layer "F.Cu") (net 3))
 (segment (start 97.25 67.25) (end 102.5 62) (width 0.5) (layer "F.Cu") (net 3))
 (segment (start 102.175 57.425) (end 102.175 58) (width 0.3) (layer "F.Cu") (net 3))
 (segment (start 97.25 68.25) (end 97.25 67.25) (width 0.5) (layer "F.Cu") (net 3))
 (segment (start 112 59.75) (end 112.25 60) (width 0.3) (layer "F.Cu") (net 3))
 (segment (start 102.175 59.425) (end 102.5 59.75) (width 0.3) (layer "F.Cu") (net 3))
 (segment (start 101.5 56.75) (end 102.175 57.425) (width 0.3) (layer "F.Cu") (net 3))
 (segment (start 100.75 56.75) (end 101.5 56.75) (width 0.3) (layer "F.Cu") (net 3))
 (segment (start 100.275 47.525) (end 99 46.25) (width 0.3) (layer "F.Cu") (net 2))
 (segment (start 100.275 55.5) (end 100.275 54.025) (width 0.3) (layer "F.Cu") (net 2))
 (segment (start 100.275 55.5) (end 100.275 47.525) (width 0.3) (layer "F.Cu") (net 2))
 (segment (start 100.275 54.025) (end 100.25 54) (width 0.3) (layer "F.Cu") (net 2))
 (segment (start 102.175 55.5) (end 102.175 54.095) (width 0.3) (layer "F.Cu") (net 5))
 (segment (start 102.175 54.095) (end 102.27 54) (width 0.3) (layer "F.Cu") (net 5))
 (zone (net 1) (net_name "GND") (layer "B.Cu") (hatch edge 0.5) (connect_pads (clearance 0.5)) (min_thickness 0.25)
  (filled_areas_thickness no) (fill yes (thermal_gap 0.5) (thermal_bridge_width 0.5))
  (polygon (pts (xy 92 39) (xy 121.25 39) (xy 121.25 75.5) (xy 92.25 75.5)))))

